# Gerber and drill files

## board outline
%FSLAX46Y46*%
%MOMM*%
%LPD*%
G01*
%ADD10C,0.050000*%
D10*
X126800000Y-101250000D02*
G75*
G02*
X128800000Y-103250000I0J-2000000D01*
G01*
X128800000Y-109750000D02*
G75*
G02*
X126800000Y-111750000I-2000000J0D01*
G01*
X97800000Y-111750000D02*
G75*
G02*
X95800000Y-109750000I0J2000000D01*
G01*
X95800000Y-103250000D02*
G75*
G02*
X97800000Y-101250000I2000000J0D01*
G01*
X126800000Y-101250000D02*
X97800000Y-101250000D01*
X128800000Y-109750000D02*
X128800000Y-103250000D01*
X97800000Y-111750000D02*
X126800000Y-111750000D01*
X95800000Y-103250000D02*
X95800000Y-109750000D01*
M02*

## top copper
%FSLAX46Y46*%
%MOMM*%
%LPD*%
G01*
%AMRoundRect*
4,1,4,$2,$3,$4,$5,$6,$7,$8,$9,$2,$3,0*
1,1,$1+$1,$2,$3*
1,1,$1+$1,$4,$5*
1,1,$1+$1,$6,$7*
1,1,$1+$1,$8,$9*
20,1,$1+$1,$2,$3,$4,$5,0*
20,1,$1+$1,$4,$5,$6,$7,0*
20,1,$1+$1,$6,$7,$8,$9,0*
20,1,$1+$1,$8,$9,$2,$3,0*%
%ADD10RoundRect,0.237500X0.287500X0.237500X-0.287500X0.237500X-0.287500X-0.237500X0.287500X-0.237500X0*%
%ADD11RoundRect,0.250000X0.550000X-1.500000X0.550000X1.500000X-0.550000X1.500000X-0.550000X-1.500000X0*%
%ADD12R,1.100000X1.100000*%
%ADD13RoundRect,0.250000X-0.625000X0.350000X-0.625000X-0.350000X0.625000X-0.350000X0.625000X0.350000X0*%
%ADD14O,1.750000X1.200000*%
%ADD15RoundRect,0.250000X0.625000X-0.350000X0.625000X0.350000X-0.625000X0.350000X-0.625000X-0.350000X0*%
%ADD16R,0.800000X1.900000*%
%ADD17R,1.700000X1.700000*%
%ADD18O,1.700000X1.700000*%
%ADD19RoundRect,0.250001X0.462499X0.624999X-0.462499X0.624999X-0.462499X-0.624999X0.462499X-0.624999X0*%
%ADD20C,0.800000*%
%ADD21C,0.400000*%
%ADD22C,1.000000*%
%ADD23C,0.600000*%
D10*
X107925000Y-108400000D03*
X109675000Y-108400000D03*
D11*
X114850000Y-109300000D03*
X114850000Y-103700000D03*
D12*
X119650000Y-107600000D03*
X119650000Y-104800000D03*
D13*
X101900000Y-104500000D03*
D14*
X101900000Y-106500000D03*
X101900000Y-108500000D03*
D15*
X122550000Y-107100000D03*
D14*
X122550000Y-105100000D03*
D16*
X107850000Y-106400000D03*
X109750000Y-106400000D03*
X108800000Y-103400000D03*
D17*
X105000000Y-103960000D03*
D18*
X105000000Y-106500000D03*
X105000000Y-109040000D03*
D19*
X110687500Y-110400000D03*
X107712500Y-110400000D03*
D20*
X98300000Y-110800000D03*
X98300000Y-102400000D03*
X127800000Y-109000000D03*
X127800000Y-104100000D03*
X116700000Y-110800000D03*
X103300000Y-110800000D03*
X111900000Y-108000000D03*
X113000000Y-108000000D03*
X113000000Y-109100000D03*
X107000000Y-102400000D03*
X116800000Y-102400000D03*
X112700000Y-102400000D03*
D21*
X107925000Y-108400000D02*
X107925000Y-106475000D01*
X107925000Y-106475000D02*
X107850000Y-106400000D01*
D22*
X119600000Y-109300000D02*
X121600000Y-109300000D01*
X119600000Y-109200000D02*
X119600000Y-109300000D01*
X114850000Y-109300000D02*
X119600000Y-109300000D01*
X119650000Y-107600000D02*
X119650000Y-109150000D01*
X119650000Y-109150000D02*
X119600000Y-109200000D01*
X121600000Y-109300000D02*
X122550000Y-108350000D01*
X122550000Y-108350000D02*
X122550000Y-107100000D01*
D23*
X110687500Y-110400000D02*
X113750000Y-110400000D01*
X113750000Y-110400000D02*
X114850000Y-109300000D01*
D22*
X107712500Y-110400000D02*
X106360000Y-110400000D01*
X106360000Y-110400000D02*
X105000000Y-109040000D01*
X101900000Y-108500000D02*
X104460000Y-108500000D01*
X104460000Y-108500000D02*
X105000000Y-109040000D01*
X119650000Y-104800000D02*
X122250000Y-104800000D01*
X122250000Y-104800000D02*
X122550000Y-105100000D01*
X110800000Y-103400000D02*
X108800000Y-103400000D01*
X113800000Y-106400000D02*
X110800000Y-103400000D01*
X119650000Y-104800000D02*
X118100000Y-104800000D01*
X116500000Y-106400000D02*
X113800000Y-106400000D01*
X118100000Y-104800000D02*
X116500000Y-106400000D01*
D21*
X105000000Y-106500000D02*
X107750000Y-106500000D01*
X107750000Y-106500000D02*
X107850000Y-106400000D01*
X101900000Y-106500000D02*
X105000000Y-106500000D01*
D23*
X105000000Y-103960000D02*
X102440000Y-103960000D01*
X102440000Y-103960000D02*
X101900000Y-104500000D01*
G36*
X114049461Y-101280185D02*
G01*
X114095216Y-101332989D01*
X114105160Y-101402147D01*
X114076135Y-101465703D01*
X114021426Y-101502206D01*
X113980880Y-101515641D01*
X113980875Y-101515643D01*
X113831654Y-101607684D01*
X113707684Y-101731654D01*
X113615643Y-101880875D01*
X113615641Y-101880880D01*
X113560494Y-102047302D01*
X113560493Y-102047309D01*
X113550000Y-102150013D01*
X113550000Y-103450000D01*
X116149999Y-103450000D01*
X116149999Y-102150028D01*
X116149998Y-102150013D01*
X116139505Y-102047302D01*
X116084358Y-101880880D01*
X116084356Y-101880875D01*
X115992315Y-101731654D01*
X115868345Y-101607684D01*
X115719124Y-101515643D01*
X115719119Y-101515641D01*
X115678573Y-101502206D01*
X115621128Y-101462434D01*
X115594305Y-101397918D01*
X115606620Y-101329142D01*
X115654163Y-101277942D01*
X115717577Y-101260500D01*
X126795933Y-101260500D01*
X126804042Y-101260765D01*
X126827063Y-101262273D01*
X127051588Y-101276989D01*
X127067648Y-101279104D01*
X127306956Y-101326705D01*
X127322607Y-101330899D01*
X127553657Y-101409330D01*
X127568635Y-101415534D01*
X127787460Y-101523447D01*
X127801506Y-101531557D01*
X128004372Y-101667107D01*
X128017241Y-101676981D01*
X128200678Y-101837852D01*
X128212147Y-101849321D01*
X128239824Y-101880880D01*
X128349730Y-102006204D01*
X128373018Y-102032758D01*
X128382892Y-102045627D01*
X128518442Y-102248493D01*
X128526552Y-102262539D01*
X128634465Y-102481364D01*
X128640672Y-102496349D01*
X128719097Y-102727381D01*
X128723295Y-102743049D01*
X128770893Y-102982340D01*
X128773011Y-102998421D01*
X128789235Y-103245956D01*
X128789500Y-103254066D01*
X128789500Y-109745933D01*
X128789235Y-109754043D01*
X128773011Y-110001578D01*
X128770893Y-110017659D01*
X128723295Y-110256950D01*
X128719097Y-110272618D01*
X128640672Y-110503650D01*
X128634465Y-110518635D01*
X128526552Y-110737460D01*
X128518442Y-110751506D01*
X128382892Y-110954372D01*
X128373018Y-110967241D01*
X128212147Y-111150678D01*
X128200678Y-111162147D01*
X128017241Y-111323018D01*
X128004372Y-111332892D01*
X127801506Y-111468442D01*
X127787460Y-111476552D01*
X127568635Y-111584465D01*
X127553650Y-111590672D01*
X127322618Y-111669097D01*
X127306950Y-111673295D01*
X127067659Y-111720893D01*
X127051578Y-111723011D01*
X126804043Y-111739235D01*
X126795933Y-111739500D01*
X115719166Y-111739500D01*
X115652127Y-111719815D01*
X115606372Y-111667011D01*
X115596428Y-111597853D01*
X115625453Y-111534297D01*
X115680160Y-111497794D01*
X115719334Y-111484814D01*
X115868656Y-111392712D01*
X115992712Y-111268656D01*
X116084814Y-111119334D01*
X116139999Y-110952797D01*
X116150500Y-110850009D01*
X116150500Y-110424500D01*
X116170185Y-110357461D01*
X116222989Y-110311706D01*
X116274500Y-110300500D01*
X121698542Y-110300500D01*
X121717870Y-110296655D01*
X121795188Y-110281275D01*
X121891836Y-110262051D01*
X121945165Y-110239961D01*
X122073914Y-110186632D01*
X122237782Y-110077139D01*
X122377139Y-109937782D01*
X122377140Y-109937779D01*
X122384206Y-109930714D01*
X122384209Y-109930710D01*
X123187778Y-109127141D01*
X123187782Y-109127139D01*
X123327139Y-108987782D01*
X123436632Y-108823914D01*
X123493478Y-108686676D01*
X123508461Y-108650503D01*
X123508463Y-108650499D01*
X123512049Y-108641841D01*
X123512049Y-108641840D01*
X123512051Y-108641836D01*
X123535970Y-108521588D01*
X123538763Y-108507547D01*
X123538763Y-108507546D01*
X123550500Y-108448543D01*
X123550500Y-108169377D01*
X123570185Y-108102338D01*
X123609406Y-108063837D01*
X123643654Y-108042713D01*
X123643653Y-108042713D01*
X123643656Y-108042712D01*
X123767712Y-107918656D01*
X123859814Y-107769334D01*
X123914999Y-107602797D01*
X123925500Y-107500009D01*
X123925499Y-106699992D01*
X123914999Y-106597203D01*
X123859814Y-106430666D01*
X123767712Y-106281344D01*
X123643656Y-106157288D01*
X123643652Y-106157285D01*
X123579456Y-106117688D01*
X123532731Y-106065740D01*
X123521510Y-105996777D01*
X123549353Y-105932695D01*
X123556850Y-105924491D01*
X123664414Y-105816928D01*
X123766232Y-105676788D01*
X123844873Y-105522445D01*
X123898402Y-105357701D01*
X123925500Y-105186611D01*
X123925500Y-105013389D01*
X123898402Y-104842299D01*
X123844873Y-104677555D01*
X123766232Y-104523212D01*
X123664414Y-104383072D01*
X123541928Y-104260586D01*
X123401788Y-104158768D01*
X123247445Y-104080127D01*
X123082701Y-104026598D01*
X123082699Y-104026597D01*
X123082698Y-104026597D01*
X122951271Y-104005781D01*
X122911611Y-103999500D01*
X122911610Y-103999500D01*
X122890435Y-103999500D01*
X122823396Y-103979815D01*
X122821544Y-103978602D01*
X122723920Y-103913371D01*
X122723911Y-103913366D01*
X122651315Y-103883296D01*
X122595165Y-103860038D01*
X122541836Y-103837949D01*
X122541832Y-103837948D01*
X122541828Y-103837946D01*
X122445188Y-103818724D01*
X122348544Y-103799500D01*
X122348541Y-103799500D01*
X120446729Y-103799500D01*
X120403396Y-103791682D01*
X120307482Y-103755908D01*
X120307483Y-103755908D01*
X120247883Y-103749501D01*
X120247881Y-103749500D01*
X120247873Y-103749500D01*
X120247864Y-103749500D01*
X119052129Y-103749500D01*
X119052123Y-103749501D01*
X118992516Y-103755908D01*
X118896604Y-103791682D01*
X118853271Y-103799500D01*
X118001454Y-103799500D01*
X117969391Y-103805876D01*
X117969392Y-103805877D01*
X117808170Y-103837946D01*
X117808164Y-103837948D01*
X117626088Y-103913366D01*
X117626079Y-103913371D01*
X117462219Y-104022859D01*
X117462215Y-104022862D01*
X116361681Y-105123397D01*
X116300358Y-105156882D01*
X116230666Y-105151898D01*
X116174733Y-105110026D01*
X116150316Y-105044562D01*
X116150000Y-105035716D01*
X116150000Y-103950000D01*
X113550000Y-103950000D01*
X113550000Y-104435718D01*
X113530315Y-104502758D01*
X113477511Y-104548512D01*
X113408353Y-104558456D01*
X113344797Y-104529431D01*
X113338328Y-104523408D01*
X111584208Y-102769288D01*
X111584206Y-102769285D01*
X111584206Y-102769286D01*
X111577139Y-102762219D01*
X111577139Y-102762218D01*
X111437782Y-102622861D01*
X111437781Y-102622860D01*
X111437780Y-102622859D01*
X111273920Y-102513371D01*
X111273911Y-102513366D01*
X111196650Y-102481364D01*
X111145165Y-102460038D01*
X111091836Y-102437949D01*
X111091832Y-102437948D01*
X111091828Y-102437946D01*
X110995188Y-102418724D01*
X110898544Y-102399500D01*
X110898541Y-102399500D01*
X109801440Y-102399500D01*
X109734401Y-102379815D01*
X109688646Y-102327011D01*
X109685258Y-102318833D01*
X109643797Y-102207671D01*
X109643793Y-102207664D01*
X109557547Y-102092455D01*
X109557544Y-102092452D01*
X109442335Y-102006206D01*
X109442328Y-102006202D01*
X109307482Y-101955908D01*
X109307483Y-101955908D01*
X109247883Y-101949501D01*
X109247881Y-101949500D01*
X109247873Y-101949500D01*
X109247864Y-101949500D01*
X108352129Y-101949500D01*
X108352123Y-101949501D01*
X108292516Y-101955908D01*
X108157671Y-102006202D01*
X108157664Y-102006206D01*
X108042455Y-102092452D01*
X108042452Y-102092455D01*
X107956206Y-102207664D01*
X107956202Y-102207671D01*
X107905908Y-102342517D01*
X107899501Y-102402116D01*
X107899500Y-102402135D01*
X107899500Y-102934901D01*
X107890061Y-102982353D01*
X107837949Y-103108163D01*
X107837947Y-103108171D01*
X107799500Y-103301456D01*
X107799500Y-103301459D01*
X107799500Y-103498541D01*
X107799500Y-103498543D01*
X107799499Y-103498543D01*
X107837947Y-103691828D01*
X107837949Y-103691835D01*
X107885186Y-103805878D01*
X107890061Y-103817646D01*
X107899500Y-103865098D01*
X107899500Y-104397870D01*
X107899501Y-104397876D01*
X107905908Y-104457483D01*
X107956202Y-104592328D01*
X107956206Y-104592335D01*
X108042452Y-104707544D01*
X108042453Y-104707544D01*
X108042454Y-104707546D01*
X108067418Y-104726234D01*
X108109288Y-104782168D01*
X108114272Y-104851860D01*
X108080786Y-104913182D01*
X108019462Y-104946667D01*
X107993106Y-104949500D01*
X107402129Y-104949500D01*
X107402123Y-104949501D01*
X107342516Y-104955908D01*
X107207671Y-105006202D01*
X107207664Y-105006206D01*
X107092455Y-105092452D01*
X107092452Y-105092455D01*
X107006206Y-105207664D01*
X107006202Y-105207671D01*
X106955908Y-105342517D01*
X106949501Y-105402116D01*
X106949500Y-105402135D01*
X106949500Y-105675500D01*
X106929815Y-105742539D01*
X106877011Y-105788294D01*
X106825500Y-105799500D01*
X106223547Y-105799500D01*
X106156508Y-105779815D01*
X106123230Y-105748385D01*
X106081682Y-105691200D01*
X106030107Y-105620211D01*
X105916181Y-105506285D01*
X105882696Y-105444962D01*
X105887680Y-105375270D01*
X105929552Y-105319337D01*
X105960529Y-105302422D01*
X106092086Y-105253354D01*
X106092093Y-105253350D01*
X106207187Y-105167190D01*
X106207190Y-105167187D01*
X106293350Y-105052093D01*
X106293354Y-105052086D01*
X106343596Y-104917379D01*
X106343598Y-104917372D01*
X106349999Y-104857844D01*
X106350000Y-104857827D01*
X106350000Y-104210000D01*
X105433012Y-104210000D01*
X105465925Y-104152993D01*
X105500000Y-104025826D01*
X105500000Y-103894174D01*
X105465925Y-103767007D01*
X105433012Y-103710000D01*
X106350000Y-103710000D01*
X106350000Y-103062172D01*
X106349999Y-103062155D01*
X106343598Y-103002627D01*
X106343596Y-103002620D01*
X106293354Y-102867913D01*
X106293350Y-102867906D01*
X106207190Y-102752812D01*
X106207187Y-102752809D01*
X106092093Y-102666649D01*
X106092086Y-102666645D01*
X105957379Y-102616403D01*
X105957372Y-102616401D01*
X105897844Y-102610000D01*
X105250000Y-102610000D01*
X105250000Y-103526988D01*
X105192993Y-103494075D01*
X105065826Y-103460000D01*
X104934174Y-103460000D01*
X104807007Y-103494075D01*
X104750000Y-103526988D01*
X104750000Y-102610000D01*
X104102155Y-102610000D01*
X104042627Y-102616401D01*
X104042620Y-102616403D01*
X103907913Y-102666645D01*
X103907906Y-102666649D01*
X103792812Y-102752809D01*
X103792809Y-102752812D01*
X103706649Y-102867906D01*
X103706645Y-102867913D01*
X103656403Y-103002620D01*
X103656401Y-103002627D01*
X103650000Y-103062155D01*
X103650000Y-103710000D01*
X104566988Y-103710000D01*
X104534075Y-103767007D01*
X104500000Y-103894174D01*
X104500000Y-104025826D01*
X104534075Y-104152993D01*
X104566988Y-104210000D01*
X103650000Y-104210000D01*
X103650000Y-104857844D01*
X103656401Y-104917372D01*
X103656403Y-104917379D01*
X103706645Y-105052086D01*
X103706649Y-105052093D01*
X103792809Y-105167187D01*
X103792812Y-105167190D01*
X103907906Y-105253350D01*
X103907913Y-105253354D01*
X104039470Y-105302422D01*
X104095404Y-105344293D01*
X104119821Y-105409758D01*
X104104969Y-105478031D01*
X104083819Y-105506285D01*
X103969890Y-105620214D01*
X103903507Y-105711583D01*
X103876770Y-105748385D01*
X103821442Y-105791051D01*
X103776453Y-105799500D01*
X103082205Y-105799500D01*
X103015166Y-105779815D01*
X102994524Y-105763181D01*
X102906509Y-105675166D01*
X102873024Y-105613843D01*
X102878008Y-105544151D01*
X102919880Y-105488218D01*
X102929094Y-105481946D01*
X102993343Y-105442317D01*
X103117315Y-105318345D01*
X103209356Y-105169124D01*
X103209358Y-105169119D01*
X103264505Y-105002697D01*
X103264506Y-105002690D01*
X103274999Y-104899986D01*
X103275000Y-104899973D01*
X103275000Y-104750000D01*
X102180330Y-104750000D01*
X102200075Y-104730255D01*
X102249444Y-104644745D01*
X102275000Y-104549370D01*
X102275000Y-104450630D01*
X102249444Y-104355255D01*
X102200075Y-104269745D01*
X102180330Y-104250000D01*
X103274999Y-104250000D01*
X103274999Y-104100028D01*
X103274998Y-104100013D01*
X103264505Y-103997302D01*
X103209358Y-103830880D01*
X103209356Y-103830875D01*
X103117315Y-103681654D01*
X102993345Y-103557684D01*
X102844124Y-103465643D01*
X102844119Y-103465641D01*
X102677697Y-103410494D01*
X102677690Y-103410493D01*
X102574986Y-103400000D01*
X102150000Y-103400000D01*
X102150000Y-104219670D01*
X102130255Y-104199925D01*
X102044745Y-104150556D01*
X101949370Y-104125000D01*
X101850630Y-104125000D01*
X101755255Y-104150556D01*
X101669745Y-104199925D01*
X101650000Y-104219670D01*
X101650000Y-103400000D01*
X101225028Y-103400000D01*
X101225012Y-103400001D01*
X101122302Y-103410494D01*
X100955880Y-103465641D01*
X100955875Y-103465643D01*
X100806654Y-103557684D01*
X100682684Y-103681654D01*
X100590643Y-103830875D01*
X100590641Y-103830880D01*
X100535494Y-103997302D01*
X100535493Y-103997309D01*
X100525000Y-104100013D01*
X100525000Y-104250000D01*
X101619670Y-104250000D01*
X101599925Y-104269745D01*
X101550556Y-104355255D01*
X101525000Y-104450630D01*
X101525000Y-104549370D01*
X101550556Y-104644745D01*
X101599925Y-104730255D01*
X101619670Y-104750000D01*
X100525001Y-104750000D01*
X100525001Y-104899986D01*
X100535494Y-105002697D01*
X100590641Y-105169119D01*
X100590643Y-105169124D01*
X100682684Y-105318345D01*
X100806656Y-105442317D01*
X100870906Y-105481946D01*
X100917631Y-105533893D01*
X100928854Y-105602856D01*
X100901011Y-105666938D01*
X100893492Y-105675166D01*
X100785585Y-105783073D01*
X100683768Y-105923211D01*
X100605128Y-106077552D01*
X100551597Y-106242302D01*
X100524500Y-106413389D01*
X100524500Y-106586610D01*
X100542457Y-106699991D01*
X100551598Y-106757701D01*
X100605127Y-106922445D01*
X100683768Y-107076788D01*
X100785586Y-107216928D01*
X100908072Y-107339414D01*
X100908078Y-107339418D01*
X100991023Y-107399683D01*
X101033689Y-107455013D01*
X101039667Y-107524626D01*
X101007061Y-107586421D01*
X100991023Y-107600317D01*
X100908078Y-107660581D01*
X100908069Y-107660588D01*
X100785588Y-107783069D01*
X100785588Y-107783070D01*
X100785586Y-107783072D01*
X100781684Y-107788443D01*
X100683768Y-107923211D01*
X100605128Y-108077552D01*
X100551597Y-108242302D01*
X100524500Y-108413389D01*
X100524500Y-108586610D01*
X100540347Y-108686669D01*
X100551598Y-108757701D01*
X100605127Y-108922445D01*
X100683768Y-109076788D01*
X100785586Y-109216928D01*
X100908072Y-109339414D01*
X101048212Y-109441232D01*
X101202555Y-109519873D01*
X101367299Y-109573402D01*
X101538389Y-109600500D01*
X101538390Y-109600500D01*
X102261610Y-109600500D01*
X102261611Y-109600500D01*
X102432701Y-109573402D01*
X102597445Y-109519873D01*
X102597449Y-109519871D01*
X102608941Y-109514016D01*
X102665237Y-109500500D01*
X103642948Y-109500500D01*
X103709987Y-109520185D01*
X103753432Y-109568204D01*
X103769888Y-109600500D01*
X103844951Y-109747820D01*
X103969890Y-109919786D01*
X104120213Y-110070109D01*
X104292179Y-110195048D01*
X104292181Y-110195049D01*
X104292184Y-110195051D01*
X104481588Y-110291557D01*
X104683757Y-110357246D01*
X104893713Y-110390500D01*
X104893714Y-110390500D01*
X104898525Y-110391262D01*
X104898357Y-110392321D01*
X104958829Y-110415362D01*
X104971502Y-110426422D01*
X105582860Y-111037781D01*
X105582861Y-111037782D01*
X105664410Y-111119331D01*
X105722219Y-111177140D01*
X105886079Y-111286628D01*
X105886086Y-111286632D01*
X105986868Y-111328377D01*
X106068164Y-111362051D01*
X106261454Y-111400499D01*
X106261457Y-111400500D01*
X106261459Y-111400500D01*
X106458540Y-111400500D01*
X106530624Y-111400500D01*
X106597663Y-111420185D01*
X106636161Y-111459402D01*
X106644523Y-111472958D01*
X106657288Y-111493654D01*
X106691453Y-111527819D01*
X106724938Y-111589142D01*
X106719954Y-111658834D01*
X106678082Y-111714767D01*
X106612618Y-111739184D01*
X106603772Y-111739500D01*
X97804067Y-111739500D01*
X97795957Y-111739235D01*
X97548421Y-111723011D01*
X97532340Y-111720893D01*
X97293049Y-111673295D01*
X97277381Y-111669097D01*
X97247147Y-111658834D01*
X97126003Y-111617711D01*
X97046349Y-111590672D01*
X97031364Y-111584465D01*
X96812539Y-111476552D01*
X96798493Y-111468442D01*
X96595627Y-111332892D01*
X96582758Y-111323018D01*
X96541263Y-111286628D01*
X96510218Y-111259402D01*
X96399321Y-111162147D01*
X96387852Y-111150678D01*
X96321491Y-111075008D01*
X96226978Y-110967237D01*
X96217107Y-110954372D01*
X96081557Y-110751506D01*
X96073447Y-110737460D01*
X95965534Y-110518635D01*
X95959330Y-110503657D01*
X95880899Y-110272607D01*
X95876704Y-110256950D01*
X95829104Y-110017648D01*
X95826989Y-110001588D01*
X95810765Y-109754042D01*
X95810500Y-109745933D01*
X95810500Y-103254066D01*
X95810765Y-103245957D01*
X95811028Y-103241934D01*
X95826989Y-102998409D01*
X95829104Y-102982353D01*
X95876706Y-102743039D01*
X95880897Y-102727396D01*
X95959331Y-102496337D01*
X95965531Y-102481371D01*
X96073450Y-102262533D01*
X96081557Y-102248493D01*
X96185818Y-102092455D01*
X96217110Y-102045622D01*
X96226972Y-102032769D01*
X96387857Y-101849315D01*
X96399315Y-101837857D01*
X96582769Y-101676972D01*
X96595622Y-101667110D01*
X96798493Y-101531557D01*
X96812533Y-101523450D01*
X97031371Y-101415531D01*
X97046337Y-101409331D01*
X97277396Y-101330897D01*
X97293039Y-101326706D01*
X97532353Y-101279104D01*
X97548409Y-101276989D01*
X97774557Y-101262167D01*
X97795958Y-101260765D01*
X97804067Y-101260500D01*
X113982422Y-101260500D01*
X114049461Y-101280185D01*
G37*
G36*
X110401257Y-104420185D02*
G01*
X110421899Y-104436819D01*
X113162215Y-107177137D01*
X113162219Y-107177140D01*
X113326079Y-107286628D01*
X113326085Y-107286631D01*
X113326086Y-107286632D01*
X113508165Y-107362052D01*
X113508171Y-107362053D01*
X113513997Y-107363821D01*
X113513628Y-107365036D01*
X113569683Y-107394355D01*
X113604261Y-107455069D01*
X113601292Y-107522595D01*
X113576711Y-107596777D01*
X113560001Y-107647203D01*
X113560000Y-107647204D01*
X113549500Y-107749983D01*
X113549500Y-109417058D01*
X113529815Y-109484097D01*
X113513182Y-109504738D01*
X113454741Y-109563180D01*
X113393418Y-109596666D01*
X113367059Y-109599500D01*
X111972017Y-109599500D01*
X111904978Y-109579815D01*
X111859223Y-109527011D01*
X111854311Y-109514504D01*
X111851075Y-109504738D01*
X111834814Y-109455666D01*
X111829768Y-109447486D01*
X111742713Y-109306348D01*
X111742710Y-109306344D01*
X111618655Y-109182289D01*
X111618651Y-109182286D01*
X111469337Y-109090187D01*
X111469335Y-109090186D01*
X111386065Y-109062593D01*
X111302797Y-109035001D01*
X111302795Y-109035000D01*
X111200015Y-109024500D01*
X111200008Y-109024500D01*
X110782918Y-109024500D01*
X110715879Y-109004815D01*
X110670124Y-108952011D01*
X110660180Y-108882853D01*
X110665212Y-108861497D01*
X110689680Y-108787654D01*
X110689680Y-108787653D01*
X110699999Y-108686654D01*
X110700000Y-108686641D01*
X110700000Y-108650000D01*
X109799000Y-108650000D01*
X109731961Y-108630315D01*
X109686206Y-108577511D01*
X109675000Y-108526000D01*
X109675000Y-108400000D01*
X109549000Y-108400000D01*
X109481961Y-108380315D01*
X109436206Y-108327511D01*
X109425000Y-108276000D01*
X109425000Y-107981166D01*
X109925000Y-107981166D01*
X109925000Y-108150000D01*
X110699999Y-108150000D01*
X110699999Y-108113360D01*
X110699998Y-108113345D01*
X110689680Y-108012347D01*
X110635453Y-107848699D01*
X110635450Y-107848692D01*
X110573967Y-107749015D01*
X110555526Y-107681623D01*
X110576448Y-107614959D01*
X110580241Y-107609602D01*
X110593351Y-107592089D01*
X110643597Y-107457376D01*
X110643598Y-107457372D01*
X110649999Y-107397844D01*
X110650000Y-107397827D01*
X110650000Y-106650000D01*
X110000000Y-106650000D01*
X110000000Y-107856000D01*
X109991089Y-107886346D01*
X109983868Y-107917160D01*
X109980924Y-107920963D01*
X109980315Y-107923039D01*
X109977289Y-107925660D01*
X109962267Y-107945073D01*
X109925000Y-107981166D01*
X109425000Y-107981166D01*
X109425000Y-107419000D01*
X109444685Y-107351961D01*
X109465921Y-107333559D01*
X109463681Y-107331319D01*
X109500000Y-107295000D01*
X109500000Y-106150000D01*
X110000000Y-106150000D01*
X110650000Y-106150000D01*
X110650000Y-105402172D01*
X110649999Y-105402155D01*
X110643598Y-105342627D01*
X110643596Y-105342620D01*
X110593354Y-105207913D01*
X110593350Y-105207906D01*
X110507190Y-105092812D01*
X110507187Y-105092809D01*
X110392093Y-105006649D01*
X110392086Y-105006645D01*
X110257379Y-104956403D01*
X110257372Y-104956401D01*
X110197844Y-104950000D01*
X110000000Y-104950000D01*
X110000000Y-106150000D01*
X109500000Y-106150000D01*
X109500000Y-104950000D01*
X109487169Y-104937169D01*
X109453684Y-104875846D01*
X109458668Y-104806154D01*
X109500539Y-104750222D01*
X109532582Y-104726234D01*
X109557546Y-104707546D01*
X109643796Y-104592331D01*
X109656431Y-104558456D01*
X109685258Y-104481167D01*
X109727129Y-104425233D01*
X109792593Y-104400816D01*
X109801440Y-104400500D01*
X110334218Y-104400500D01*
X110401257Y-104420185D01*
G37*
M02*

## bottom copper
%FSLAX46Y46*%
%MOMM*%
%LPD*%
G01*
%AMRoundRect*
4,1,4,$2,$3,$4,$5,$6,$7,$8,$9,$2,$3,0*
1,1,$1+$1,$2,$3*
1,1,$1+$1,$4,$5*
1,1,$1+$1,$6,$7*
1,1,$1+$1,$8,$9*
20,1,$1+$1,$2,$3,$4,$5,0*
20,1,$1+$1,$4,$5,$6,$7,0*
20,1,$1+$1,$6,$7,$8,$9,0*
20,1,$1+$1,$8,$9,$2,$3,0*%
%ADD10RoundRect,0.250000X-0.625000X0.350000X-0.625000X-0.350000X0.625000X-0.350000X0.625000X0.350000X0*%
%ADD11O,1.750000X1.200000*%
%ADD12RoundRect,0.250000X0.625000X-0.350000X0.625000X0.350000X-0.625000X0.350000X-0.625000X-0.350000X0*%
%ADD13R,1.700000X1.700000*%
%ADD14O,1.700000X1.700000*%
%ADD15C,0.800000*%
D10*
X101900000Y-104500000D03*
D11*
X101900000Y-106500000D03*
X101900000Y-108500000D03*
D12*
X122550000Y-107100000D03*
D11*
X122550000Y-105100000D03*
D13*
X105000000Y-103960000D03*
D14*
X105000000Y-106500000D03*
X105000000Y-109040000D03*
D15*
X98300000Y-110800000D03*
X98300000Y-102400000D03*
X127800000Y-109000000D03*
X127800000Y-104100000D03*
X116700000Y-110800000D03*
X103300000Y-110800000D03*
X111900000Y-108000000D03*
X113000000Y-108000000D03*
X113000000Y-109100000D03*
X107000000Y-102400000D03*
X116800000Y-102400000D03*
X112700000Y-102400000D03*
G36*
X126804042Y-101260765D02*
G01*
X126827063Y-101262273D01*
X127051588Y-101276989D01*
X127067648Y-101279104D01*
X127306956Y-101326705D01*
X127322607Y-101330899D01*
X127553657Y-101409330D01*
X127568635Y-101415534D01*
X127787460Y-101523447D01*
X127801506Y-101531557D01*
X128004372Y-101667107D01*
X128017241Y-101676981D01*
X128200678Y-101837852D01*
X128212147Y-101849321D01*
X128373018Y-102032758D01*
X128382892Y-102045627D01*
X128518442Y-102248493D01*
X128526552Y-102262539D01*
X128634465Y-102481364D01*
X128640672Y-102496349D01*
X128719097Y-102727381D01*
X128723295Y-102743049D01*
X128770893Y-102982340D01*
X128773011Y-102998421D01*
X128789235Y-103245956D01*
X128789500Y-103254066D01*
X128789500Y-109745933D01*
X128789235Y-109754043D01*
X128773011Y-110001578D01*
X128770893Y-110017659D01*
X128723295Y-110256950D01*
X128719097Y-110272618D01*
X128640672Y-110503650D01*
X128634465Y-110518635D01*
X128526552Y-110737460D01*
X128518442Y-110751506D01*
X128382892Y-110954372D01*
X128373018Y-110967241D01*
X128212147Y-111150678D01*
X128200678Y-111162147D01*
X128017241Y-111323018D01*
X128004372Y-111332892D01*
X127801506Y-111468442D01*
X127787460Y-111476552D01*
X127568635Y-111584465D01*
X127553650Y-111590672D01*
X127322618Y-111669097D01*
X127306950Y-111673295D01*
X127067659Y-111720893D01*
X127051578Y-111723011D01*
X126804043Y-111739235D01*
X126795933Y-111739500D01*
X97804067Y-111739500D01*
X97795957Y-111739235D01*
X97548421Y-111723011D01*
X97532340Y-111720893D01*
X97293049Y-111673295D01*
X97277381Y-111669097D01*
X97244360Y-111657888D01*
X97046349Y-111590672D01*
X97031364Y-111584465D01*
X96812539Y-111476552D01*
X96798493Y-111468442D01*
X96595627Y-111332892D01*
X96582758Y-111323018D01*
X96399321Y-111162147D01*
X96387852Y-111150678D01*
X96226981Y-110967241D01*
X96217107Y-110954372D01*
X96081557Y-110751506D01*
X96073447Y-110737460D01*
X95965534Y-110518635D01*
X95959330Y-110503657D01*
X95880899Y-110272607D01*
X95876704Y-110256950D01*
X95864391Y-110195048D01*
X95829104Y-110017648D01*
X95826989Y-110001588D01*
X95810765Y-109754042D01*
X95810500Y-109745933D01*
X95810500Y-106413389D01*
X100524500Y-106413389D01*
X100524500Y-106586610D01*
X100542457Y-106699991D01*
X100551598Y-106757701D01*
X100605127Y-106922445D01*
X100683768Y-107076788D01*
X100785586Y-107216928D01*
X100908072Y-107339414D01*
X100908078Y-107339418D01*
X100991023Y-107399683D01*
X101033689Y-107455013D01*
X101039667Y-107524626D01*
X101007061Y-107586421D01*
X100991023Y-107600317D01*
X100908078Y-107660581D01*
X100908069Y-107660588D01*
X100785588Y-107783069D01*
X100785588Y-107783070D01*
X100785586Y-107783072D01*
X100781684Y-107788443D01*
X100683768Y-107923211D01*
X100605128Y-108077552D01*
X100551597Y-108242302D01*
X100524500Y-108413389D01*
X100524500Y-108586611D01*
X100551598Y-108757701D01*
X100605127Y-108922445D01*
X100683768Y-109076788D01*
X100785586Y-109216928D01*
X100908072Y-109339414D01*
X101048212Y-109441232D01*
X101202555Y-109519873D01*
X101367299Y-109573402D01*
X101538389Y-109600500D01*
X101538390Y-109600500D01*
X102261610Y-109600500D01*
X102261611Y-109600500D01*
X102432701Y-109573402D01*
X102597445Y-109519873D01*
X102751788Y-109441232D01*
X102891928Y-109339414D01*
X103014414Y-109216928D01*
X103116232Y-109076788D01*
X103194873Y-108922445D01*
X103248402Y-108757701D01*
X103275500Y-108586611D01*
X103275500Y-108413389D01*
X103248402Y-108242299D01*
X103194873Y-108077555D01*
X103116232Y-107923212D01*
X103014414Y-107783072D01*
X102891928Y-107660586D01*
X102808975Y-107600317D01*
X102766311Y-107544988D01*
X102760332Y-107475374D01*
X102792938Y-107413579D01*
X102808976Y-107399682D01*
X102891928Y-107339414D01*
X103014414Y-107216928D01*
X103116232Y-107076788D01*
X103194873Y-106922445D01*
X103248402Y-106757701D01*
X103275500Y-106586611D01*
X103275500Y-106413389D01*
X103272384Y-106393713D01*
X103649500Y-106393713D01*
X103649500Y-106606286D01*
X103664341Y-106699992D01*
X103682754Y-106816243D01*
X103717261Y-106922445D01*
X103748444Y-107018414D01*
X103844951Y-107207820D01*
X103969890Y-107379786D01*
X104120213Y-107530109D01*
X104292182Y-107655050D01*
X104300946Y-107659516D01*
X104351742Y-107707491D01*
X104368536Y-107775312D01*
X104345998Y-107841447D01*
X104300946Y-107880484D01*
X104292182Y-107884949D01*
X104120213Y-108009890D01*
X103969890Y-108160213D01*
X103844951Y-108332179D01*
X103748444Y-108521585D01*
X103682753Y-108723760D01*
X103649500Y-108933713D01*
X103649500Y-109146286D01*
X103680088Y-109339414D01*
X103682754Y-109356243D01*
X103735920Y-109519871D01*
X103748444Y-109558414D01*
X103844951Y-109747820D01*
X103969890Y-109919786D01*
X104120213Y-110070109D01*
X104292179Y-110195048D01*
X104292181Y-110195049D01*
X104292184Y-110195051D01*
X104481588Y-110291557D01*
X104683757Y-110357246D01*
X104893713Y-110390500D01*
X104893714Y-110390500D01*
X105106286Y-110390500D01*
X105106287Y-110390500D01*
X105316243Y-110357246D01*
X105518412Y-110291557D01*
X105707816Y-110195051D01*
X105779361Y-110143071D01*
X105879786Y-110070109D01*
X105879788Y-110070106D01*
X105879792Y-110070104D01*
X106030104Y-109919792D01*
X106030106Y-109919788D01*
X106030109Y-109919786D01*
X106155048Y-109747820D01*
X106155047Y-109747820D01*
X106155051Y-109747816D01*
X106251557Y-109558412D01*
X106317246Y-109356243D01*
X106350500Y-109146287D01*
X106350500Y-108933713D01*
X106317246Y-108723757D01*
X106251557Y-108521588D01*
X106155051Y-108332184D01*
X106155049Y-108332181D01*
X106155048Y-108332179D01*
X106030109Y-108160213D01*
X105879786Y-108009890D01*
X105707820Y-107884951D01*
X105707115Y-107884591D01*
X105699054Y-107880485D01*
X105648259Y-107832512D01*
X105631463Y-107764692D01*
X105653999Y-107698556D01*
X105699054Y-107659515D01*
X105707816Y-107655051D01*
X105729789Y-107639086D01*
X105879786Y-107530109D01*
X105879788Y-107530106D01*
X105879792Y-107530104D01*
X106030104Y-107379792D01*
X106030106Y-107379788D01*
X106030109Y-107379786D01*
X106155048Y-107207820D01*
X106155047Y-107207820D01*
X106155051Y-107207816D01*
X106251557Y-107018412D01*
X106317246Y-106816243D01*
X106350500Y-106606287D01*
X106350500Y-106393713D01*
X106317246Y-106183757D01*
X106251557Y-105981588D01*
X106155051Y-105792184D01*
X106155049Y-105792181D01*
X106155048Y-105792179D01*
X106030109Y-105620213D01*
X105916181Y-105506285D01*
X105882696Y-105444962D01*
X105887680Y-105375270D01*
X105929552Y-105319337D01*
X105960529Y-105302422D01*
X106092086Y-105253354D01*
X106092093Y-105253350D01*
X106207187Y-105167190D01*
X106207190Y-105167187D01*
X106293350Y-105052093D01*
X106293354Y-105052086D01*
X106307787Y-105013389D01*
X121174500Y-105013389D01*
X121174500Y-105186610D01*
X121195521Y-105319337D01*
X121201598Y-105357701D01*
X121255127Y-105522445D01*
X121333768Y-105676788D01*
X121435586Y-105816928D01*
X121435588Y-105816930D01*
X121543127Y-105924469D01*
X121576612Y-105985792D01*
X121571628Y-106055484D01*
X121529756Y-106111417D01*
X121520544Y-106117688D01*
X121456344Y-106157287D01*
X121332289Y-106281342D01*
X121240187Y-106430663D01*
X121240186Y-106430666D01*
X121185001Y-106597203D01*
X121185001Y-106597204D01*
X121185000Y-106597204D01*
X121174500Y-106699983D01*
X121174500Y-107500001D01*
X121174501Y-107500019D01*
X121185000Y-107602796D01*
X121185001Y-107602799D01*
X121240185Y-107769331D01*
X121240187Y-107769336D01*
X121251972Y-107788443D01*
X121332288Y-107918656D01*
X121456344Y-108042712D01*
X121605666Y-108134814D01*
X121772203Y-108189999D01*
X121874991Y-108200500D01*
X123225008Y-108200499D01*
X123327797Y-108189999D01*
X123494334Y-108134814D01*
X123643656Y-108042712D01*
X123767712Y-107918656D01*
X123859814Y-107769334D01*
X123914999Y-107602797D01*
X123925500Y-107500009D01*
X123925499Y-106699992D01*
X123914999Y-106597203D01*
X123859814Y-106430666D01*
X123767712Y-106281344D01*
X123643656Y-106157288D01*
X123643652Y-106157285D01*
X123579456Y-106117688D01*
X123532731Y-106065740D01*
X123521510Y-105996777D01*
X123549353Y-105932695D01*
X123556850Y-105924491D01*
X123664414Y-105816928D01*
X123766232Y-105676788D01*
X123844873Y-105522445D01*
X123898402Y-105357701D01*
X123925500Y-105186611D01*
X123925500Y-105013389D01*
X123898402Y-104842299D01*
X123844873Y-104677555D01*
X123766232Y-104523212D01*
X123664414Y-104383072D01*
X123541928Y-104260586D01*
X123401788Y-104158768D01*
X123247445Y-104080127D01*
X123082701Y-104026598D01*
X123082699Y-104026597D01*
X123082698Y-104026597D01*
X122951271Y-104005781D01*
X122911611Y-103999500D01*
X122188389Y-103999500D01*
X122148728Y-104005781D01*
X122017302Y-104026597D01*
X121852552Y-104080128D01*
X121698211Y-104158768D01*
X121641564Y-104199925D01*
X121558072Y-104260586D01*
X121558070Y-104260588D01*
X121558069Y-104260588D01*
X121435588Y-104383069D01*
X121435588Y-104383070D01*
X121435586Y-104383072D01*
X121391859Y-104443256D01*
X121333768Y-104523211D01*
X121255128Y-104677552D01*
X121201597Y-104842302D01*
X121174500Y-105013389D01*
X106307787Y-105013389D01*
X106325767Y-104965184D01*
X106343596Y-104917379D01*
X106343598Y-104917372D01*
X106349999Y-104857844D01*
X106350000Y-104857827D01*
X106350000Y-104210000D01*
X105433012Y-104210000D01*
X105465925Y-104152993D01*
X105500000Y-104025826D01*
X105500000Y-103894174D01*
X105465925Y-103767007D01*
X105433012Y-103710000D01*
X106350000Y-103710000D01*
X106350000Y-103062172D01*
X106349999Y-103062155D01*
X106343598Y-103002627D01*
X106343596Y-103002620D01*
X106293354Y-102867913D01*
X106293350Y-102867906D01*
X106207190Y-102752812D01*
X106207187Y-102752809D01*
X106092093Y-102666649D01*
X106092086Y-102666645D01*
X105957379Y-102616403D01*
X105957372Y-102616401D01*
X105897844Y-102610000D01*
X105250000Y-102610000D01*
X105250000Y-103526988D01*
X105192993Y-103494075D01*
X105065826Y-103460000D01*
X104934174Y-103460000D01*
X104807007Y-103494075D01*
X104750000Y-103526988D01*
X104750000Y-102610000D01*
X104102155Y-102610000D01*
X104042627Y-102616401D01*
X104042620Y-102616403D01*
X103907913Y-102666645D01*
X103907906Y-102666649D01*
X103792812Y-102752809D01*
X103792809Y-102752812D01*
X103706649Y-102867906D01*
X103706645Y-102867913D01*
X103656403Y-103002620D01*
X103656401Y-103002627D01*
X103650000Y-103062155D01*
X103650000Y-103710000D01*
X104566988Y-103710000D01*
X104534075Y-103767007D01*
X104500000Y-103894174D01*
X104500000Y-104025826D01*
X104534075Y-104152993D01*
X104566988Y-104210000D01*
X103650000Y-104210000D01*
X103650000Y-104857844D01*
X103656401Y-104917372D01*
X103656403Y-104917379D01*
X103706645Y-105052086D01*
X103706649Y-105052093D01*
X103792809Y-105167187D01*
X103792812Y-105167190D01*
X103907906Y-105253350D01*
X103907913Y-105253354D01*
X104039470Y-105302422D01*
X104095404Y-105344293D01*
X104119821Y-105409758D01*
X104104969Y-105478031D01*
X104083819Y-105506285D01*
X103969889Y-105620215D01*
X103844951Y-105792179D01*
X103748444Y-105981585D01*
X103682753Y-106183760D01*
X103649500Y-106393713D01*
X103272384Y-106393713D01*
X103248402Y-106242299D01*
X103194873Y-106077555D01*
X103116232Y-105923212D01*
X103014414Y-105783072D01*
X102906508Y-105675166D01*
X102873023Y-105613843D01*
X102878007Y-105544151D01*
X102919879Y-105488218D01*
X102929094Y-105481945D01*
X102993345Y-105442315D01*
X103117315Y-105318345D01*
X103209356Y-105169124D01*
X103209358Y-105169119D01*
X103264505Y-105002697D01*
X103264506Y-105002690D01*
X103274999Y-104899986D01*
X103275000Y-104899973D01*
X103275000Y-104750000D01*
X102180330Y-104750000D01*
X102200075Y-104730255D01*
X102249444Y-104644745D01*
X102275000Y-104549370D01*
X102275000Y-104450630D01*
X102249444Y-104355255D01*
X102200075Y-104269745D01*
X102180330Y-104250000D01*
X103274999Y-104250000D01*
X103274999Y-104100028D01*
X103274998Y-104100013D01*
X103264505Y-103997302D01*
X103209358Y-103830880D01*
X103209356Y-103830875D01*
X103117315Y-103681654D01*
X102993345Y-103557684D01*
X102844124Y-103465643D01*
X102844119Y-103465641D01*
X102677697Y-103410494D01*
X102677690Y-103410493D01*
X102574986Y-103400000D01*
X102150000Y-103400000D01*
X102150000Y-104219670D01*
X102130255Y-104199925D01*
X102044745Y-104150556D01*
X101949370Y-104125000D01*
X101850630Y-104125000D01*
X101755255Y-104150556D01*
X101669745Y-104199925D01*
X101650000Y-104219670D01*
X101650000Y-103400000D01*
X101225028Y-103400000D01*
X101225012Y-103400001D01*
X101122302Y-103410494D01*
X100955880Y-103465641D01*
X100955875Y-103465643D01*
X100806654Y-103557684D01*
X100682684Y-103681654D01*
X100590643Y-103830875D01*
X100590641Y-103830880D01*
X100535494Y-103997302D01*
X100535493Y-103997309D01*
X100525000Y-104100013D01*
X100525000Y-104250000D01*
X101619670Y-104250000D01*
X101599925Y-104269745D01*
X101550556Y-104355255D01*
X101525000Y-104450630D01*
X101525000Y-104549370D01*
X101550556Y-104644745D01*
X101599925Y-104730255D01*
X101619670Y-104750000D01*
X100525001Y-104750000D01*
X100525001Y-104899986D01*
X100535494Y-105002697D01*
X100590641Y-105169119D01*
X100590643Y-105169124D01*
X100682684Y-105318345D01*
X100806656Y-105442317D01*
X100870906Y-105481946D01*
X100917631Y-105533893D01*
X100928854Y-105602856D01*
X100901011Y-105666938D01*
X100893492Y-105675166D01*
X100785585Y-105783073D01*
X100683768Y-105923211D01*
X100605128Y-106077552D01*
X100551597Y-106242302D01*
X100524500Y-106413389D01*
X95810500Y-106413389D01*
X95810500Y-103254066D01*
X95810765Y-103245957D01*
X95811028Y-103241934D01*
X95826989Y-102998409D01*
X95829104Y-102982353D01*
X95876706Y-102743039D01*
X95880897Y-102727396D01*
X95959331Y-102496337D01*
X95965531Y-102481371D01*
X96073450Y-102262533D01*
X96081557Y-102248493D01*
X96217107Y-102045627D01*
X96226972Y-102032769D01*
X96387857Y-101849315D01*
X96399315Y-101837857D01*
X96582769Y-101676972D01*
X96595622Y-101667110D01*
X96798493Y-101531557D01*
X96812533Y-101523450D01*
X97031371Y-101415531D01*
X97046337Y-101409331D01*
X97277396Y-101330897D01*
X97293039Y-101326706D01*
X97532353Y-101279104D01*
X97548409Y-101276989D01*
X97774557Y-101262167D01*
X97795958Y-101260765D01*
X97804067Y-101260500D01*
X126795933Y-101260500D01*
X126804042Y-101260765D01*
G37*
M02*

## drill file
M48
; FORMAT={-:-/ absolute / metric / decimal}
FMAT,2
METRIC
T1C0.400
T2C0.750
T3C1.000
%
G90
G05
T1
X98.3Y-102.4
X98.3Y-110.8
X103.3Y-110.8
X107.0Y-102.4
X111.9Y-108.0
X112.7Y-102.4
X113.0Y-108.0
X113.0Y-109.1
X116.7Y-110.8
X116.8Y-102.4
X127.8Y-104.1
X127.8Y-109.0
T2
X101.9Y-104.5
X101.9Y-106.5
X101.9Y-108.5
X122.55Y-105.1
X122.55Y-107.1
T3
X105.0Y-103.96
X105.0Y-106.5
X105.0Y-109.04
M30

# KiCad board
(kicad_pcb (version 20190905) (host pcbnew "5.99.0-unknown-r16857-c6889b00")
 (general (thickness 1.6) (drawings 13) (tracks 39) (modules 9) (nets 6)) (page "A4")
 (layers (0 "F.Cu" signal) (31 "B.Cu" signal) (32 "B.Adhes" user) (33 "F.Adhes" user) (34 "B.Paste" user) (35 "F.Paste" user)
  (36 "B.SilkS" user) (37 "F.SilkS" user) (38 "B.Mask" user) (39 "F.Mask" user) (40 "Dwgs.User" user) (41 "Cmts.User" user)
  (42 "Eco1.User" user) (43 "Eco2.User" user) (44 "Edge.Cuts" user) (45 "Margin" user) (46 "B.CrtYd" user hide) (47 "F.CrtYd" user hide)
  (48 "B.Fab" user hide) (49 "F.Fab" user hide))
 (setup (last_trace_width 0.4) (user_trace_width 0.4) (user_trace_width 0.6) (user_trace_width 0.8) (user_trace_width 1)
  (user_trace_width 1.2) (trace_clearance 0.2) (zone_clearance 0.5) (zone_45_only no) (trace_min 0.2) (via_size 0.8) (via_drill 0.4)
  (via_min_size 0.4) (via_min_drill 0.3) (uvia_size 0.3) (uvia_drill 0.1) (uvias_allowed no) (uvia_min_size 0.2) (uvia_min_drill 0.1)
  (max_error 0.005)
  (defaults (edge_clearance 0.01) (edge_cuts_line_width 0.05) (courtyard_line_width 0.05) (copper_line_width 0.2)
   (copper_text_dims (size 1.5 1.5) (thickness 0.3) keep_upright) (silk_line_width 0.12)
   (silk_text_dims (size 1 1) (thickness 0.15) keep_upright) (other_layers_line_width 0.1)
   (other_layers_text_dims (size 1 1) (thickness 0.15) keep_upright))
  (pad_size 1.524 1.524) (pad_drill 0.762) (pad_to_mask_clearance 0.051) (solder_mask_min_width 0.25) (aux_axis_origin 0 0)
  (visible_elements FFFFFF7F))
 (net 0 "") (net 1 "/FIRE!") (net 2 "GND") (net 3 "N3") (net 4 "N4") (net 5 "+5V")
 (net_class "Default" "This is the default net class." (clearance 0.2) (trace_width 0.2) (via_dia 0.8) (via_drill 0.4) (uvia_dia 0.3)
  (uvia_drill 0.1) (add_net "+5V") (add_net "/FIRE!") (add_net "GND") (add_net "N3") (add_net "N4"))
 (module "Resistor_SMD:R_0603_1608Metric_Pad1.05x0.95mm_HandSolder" (layer "F.Cu") (at 108.8 108.4 180)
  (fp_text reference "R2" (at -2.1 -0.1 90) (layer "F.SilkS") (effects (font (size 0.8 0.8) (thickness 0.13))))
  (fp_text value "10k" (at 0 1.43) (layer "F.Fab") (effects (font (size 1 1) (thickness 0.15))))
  (pad "2" smd roundrect (at 0.875 0 180) (size 1.05 0.95) (layers "F.Cu" "F.Paste" "F.Mask") (roundrect_rratio 0.25) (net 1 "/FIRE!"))
  (pad "1" smd roundrect (at -0.875 0 180) (size 1.05 0.95) (layers "F.Cu" "F.Paste" "F.Mask") (roundrect_rratio 0.25) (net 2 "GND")))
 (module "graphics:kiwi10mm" (layer "B.Cu") (at 113.55 107 180)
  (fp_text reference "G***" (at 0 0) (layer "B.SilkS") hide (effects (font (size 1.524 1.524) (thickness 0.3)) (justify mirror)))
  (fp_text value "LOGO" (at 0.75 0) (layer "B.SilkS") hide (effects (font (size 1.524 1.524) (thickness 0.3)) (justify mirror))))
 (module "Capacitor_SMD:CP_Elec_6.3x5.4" (layer "F.Cu") (at 114.85 106.5 90)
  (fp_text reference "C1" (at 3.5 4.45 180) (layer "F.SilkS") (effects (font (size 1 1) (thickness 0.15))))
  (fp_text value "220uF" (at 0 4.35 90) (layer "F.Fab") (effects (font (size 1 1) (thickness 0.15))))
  (pad "1" smd roundrect (at -2.8 0 90) (size 3.5 1.6) (layers "F.Cu" "F.Paste" "F.Mask") (roundrect_rratio 0.15625) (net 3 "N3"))
  (pad "2" smd roundrect (at 2.8 0 90) (size 3.5 1.6) (layers "F.Cu" "F.Paste" "F.Mask") (roundrect_rratio 0.15625) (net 2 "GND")))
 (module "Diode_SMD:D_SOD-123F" (layer "F.Cu") (at 119.65 106.2 90)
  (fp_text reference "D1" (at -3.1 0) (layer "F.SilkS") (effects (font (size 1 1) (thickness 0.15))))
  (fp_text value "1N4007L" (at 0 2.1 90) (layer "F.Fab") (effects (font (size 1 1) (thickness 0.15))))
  (pad "1" smd rect (at -1.4 0 90) (size 1.1 1.1) (layers "F.Cu" "F.Paste" "F.Mask") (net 3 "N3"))
  (pad "2" smd rect (at 1.4 0 90) (size 1.1 1.1) (layers "F.Cu" "F.Paste" "F.Mask") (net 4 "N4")))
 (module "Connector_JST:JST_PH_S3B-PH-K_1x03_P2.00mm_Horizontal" (layer "F.Cu") (at 101.9 104.5 270)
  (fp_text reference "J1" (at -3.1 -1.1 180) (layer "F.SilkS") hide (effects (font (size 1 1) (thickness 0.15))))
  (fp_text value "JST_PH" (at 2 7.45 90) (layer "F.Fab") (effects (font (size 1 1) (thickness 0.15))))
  (pad "1" thru_hole roundrect (at 0 0 270) (size 1.2 1.75) (drill 0.75) (layers *.Cu *.Mask) (roundrect_rratio 0.208333) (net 2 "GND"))
  (pad "2" thru_hole oval (at 2 0 270) (size 1.2 1.75) (drill 0.75) (layers *.Cu *.Mask) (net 1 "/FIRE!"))
  (pad "3" thru_hole oval (at 4 0 270) (size 1.2 1.75) (drill 0.75) (layers *.Cu *.Mask) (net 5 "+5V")))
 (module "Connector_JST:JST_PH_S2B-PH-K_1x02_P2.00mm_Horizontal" (layer "F.Cu") (at 122.55 107.1 90)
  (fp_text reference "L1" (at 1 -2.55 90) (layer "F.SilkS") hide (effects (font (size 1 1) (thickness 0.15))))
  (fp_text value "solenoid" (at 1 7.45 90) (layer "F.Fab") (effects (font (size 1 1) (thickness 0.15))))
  (pad "1" thru_hole roundrect (at 0 0 90) (size 1.2 1.75) (drill 0.75) (layers *.Cu *.Mask) (roundrect_rratio 0.208333) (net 3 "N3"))
  (pad "2" thru_hole oval (at 2 0 90) (size 1.2 1.75) (drill 0.75) (layers *.Cu *.Mask) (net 4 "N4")))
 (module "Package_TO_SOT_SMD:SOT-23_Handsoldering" (layer "F.Cu") (at 108.8 104.9 90)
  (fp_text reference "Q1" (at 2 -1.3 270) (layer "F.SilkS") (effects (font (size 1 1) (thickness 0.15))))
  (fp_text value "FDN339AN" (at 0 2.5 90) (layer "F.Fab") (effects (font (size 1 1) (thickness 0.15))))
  (pad "1" smd rect (at -1.5 -0.95 90) (size 1.9 0.8) (layers "F.Cu" "F.Paste" "F.Mask") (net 1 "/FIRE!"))
  (pad "2" smd rect (at -1.5 0.95 90) (size 1.9 0.8) (layers "F.Cu" "F.Paste" "F.Mask") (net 2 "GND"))
  (pad "3" smd rect (at 1.5 0 90) (size 1.9 0.8) (layers "F.Cu" "F.Paste" "F.Mask") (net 4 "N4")))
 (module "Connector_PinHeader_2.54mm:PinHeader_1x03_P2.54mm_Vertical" (layer "F.Cu") (at 105 103.96)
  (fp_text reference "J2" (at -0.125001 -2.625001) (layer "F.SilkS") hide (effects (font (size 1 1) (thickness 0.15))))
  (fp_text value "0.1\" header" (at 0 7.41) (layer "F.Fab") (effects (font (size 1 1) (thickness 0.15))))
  (pad "1" thru_hole rect (at 0 0) (size 1.7 1.7) (drill 1) (layers *.Cu *.Mask) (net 2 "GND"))
  (pad "2" thru_hole oval (at 0 2.54) (size 1.7 1.7) (drill 1) (layers *.Cu *.Mask) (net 1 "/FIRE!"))
  (pad "3" thru_hole oval (at 0 5.08) (size 1.7 1.7) (drill 1) (layers *.Cu *.Mask) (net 5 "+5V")))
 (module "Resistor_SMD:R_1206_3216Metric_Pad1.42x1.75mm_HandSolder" (layer "F.Cu") (at 109.2 110.4 180)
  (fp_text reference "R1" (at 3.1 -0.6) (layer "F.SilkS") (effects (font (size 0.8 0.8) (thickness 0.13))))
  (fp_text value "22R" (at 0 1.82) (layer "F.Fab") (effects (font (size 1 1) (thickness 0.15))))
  (pad "1" smd roundrect (at -1.4875 0 180) (size 1.425 1.75) (layers "F.Cu" "F.Paste" "F.Mask") (roundrect_rratio 0.175439) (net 3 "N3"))
  (pad "2" smd roundrect (at 1.4875 0 180) (size 1.425 1.75) (layers "F.Cu" "F.Paste" "F.Mask") (roundrect_rratio 0.175439) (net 5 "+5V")))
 (gr_arc (start 126.8 103.25) (end 128.8 103.25) (angle -90) (layer "Edge.Cuts") (width 0.05))
 (gr_arc (start 126.8 109.75) (end 126.8 111.75) (angle -90) (layer "Edge.Cuts") (width 0.05))
 (gr_arc (start 97.8 109.75) (end 95.8 109.75) (angle -90) (layer "Edge.Cuts") (width 0.05))
 (gr_arc (start 97.8 103.25) (end 97.8 101.25) (angle -90) (layer "Edge.Cuts") (width 0.05))
 (gr_line (start 126.8 101.25) (end 97.8 101.25) (layer "Edge.Cuts") (width 0.05))
 (gr_line (start 128.8 109.75) (end 128.8 103.25) (layer "Edge.Cuts") (width 0.05))
 (gr_line (start 97.8 111.75) (end 126.8 111.75) (layer "Edge.Cuts") (width 0.05))
 (gr_line (start 95.8 103.25) (end 95.8 109.75) (layer "Edge.Cuts") (width 0.05))
 (via (at 98.3 110.8) (size 0.8) (drill 0.4) (layers "F.Cu" "B.Cu") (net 2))
 (via (at 98.3 102.4) (size 0.8) (drill 0.4) (layers "F.Cu" "B.Cu") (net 2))
 (via (at 127.8 109) (size 0.8) (drill 0.4) (layers "F.Cu" "B.Cu") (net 2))
 (via (at 127.8 104.1) (size 0.8) (drill 0.4) (layers "F.Cu" "B.Cu") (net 2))
 (via (at 116.7 110.8) (size 0.8) (drill 0.4) (layers "F.Cu" "B.Cu") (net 2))
 (via (at 103.3 110.8) (size 0.8) (drill 0.4) (layers "F.Cu" "B.Cu") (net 2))
 (via (at 111.9 108) (size 0.8) (drill 0.4) (layers "F.Cu" "B.Cu") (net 2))
 (via (at 113 108) (size 0.8) (drill 0.4) (layers "F.Cu" "B.Cu") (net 2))
 (via (at 113 109.1) (size 0.8) (drill 0.4) (layers "F.Cu" "B.Cu") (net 2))
 (segment (start 107.925 108.4) (end 107.925 106.475) (width 0.4) (layer "F.Cu") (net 1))
 (segment (start 107.925 106.475) (end 107.85 106.4) (width 0.4) (layer "F.Cu") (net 1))
 (segment (start 119.6 109.3) (end 121.6 109.3) (width 1) (layer "F.Cu") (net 3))
 (segment (start 119.6 109.2) (end 119.6 109.3) (width 1) (layer "F.Cu") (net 3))
 (segment (start 114.85 109.3) (end 119.6 109.3) (width 1) (layer "F.Cu") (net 3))
 (segment (start 119.65 107.6) (end 119.65 109.15) (width 1) (layer "F.Cu") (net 3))
 (segment (start 119.65 109.15) (end 119.6 109.2) (width 1) (layer "F.Cu") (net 3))
 (segment (start 121.6 109.3) (end 122.55 108.35) (width 1) (layer "F.Cu") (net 3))
 (segment (start 122.55 108.35) (end 122.55 107.1) (width 1) (layer "F.Cu") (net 3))
 (segment (start 110.6875 110.4) (end 113.75 110.4) (width 0.6) (layer "F.Cu") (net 3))
 (segment (start 113.75 110.4) (end 114.85 109.3) (width 0.6) (layer "F.Cu") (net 3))
 (segment (start 107.7125 110.4) (end 106.36 110.4) (width 1) (layer "F.Cu") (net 5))
 (segment (start 106.36 110.4) (end 105 109.04) (width 1) (layer "F.Cu") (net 5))
 (segment (start 101.9 108.5) (end 104.46 108.5) (width 1) (layer "F.Cu") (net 5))
 (segment (start 104.46 108.5) (end 105 109.04) (width 1) (layer "F.Cu") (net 5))
 (via (at 107 102.4) (size 0.8) (drill 0.4) (layers "F.Cu" "B.Cu") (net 2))
 (via (at 116.8 102.4) (size 0.8) (drill 0.4) (layers "F.Cu" "B.Cu") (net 2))
 (via (at 112.7 102.4) (size 0.8) (drill 0.4) (layers "F.Cu" "B.Cu") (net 2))
 (segment (start 119.65 104.8) (end 122.25 104.8) (width 1) (layer "F.Cu") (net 4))
 (segment (start 122.25 104.8) (end 122.55 105.1) (width 1) (layer "F.Cu") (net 4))
 (segment (start 110.8 103.4) (end 108.8 103.4) (width 1) (layer "F.Cu") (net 4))
 (segment (start 113.8 106.4) (end 110.8 103.4) (width 1) (layer "F.Cu") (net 4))
 (segment (start 119.65 104.8) (end 118.1 104.8) (width 1) (layer "F.Cu") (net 4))
 (segment (start 116.5 106.4) (end 113.8 106.4) (width 1) (layer "F.Cu") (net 4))
 (segment (start 118.1 104.8) (end 116.5 106.4) (width 1) (layer "F.Cu") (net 4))
 (segment (start 105 106.5) (end 107.75 106.5) (width 0.4) (layer "F.Cu") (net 1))
 (segment (start 107.75 106.5) (end 107.85 106.4) (width 0.4) (layer "F.Cu") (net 1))
 (segment (start 101.9 106.5) (end 105 106.5) (width 0.4) (layer "F.Cu") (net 1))
 (segment (start 105 103.96) (end 102.44 103.96) (width 0.6) (layer "F.Cu") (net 2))
 (segment (start 102.44 103.96) (end 101.9 104.5) (width 0.6) (layer "F.Cu") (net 2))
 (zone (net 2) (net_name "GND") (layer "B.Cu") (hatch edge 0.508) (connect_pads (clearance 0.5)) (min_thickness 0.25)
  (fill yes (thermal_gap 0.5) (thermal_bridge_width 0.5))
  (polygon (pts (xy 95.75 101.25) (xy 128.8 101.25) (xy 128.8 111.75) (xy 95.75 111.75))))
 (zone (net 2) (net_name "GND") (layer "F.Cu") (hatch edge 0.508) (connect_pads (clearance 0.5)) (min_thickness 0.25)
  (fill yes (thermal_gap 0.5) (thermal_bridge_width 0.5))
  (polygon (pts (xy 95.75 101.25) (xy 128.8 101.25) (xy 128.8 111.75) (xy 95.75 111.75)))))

